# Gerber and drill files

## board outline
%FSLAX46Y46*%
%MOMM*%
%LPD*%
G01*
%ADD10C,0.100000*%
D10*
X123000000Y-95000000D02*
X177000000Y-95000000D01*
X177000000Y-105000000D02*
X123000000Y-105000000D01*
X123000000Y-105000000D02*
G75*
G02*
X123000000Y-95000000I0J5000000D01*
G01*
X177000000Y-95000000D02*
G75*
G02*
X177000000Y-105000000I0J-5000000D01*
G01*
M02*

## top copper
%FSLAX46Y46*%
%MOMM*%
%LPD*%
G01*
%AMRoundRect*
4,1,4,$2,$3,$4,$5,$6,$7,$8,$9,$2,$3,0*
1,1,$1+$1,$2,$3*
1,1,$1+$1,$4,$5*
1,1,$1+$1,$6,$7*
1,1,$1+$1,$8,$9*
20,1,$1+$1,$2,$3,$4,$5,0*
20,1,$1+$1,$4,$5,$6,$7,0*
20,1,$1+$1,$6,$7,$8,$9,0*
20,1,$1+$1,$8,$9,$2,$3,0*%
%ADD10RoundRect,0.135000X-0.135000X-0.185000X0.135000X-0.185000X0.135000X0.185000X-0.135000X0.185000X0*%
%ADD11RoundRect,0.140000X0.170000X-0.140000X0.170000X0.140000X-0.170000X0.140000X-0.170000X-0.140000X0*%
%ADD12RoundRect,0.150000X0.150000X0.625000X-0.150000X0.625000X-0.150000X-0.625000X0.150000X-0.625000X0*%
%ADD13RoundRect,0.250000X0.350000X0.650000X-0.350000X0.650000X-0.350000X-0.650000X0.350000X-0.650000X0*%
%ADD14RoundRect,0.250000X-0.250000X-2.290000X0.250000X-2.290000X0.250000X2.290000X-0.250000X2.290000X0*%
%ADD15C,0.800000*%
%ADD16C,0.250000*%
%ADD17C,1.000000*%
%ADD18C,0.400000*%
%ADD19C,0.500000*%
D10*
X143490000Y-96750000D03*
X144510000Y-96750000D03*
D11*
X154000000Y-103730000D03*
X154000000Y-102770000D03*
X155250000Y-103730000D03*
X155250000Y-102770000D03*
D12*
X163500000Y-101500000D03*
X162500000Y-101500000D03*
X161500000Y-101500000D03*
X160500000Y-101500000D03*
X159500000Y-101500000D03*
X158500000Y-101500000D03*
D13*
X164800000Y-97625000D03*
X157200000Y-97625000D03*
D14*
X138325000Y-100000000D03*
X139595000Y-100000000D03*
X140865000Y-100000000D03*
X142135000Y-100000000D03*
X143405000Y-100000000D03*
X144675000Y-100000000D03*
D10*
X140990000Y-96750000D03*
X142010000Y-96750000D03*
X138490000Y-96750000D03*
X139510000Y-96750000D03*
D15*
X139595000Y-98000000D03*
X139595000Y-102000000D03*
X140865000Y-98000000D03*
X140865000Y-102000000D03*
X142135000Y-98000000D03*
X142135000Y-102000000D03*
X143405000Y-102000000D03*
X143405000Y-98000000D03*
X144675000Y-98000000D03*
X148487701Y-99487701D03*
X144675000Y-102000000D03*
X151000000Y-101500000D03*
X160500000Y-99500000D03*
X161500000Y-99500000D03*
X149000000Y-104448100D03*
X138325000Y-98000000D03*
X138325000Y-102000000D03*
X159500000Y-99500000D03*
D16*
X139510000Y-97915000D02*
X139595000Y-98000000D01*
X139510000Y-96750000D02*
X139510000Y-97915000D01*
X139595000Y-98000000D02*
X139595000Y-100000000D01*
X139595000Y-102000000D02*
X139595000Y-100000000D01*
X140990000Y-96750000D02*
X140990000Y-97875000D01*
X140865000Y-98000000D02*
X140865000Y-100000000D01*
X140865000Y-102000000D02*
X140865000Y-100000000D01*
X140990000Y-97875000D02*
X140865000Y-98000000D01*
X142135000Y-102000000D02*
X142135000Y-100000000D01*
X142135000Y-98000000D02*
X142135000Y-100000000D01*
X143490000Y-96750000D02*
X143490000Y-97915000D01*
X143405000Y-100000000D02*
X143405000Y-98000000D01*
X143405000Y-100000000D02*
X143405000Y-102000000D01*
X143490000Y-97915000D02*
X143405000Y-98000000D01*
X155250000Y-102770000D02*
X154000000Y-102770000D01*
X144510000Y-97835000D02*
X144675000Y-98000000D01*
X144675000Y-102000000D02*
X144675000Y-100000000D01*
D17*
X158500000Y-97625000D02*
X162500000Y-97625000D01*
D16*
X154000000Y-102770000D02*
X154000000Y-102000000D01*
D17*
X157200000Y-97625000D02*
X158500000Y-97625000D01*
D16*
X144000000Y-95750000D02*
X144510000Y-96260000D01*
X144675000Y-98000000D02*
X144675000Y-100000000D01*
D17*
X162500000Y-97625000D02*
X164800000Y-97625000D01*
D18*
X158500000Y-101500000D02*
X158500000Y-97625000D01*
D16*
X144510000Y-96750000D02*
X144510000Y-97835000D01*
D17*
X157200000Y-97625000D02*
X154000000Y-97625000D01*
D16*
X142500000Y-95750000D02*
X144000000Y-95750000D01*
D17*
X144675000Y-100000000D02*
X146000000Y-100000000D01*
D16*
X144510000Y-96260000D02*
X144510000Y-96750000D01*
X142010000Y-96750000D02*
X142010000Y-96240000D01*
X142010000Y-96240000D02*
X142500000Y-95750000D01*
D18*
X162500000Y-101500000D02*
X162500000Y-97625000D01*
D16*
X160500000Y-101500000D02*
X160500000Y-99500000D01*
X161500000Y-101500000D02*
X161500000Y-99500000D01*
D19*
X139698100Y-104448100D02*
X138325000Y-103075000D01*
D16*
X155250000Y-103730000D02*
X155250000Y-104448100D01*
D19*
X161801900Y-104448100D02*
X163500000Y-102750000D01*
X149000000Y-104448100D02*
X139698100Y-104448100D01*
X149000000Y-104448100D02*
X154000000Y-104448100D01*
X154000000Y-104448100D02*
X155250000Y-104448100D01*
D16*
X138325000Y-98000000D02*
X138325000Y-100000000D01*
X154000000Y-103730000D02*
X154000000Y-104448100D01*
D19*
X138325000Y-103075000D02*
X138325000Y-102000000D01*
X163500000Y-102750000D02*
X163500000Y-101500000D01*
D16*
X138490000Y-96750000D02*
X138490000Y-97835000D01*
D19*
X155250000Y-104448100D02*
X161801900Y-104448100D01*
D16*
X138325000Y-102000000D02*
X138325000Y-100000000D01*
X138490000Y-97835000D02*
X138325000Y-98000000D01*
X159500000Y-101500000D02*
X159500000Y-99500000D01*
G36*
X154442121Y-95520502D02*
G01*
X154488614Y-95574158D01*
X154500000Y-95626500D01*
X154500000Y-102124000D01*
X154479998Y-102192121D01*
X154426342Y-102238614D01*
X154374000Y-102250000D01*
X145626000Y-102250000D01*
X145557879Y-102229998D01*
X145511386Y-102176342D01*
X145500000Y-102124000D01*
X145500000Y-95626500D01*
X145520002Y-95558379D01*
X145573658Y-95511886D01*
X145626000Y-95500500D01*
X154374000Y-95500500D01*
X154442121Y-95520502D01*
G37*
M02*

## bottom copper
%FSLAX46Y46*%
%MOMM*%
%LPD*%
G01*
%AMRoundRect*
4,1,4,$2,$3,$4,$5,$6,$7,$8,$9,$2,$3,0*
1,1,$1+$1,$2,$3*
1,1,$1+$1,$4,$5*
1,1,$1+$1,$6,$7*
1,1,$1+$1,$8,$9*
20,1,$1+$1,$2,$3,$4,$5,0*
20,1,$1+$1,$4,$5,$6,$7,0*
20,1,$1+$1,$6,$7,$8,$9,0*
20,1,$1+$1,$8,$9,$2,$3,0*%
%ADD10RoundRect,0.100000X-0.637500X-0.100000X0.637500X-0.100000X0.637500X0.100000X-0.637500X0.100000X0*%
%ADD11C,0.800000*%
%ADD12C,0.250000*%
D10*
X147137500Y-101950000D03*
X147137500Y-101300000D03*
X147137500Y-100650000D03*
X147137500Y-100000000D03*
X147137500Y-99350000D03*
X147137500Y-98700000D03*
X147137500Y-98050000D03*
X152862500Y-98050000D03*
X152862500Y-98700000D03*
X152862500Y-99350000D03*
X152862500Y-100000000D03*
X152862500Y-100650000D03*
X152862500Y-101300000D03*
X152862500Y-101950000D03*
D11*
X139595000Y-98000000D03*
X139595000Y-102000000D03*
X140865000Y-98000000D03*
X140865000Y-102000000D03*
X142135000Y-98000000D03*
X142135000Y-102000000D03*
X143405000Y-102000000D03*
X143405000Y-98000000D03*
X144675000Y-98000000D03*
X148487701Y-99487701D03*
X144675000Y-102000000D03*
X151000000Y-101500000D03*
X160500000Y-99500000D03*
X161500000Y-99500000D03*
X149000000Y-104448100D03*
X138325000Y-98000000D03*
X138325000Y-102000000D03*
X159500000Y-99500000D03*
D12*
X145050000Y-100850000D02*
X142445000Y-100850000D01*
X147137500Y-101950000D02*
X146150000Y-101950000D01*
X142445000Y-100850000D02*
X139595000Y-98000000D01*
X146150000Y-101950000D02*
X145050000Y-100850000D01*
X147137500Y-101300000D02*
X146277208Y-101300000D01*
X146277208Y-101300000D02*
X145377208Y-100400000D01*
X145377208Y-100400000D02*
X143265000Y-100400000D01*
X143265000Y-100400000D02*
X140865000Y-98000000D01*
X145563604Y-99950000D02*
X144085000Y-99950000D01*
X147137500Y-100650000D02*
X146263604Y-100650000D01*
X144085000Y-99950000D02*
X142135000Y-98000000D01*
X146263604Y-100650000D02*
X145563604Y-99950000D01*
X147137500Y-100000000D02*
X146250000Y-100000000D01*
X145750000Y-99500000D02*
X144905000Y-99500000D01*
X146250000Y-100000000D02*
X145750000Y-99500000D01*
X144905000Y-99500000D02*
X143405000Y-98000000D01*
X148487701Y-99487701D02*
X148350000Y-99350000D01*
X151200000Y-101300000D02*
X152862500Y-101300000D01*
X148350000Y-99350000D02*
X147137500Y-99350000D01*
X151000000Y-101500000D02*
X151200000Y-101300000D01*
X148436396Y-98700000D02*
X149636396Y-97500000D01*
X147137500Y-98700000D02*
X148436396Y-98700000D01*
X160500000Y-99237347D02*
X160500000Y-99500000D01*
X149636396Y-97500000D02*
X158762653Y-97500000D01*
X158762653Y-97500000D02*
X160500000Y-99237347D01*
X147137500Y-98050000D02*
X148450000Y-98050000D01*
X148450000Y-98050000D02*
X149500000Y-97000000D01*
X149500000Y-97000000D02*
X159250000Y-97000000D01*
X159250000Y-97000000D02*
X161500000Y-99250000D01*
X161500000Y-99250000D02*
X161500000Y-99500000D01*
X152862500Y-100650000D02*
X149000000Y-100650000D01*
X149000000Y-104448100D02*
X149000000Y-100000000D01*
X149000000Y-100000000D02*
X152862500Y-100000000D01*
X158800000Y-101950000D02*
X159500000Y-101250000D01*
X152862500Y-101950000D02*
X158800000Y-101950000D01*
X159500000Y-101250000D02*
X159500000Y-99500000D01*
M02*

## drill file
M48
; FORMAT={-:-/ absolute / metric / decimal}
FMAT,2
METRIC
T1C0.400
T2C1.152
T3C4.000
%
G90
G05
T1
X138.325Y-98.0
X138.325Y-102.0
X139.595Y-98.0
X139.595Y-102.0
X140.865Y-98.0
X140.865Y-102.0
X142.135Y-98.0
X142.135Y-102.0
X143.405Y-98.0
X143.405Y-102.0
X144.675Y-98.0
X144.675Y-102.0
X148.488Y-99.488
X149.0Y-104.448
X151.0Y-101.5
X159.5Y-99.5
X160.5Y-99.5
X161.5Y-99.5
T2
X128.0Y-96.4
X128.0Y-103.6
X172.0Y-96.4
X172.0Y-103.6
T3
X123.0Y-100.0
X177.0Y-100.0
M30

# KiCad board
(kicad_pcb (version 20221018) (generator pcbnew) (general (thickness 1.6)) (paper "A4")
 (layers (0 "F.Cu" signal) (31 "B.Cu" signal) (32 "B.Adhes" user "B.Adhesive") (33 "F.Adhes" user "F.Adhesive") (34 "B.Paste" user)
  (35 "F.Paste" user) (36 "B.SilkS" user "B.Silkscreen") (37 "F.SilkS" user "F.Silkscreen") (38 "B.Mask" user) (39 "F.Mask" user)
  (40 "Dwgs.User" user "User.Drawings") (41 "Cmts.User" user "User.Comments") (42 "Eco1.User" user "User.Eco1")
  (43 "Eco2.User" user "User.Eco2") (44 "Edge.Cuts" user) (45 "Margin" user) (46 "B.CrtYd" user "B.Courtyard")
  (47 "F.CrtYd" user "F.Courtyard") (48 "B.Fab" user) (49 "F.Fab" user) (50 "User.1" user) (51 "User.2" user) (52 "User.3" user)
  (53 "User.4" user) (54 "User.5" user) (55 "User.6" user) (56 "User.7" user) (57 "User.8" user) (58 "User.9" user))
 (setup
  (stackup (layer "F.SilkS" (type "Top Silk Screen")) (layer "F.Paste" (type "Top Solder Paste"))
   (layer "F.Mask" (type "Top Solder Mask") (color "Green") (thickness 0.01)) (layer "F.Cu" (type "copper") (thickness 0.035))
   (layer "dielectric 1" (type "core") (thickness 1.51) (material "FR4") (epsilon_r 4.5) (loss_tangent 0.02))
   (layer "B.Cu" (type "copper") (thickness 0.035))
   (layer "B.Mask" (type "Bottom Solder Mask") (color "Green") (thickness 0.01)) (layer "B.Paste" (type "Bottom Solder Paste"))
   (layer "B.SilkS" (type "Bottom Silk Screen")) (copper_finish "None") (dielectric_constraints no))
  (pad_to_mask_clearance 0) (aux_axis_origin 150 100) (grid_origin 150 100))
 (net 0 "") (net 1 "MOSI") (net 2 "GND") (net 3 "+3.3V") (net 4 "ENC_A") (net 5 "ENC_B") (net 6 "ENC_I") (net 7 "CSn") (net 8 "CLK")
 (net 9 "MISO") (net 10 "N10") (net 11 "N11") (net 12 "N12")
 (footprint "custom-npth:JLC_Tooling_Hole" (layer "F.Cu") (at 128 103.6)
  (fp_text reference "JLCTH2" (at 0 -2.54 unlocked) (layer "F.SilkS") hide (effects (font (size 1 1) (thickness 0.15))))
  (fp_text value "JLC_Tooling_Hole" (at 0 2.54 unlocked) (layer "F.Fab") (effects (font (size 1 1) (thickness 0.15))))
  (pad "" np_thru_hole circle (at 0 0) (size 1.3 1.3) (drill 1.152) (layers "*.Mask") (solder_mask_margin 0.074) (clearance 0.248)
   (zone_connect 0)))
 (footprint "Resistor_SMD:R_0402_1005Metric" (layer "F.Cu") (at 144 96.75)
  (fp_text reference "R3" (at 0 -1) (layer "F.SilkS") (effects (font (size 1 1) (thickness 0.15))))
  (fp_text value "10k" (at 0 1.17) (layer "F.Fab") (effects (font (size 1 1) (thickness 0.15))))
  (pad "1" smd roundrect (at -0.51 0) (size 0.54 0.64) (layers "F.Cu" "F.Paste" "F.Mask") (roundrect_rratio 0.25) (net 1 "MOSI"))
  (pad "2" smd roundrect (at 0.51 0) (size 0.54 0.64) (layers "F.Cu" "F.Paste" "F.Mask") (roundrect_rratio 0.25) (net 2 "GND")))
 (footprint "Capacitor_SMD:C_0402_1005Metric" (layer "F.Cu") (at 154 103.25 90)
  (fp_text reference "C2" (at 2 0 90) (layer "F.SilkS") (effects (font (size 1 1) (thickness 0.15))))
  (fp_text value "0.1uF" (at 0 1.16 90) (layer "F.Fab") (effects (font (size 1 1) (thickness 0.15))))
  (pad "1" smd roundrect (at -0.48 0 90) (size 0.56 0.62) (layers "F.Cu" "F.Paste" "F.Mask") (roundrect_rratio 0.25) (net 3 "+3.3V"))
  (pad "2" smd roundrect (at 0.48 0 90) (size 0.56 0.62) (layers "F.Cu" "F.Paste" "F.Mask") (roundrect_rratio 0.25) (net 2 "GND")))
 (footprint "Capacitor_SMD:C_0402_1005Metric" (layer "F.Cu") (at 155.25 103.25 90)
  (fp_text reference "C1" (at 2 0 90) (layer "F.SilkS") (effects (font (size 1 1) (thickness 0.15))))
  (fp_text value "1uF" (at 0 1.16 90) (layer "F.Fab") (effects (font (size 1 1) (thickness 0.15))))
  (pad "1" smd roundrect (at -0.48 0 90) (size 0.56 0.62) (layers "F.Cu" "F.Paste" "F.Mask") (roundrect_rratio 0.25) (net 3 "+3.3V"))
  (pad "2" smd roundrect (at 0.48 0 90) (size 0.56 0.62) (layers "F.Cu" "F.Paste" "F.Mask") (roundrect_rratio 0.25) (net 2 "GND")))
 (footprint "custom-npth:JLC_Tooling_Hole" (layer "F.Cu") (at 128 96.4)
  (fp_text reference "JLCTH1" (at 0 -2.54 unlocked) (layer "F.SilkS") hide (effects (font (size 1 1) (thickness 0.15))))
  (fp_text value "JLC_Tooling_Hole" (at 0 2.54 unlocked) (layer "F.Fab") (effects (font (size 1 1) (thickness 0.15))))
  (pad "" np_thru_hole circle (at 0 0) (size 1.3 1.3) (drill 1.152) (layers "*.Mask") (solder_mask_margin 0.074) (clearance 0.248)
   (zone_connect 0)))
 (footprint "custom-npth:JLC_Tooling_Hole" (layer "F.Cu") (at 172 103.6)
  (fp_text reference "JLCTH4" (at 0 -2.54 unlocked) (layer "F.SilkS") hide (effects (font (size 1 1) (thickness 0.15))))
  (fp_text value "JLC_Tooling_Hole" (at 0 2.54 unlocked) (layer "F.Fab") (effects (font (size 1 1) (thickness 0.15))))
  (pad "" np_thru_hole circle (at 0 0) (size 1.3 1.3) (drill 1.152) (layers "*.Mask") (solder_mask_margin 0.074) (clearance 0.248)
   (zone_connect 0)))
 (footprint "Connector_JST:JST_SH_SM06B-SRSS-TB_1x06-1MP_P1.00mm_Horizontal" (layer "F.Cu") (at 161 99.5 180)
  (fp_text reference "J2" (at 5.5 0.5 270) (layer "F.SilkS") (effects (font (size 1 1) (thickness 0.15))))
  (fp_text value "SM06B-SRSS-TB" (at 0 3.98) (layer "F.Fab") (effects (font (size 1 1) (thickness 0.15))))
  (pad "1" smd roundrect (at -2.5 -2 180) (size 0.6 1.55) (layers "F.Cu" "F.Paste" "F.Mask") (roundrect_rratio 0.25) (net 3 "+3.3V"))
  (pad "2" smd roundrect (at -1.5 -2 180) (size 0.6 1.55) (layers "F.Cu" "F.Paste" "F.Mask") (roundrect_rratio 0.25) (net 2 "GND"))
  (pad "3" smd roundrect (at -0.5 -2 180) (size 0.6 1.55) (layers "F.Cu" "F.Paste" "F.Mask") (roundrect_rratio 0.25) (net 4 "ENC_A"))
  (pad "4" smd roundrect (at 0.5 -2 180) (size 0.6 1.55) (layers "F.Cu" "F.Paste" "F.Mask") (roundrect_rratio 0.25) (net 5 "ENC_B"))
  (pad "5" smd roundrect (at 1.5 -2 180) (size 0.6 1.55) (layers "F.Cu" "F.Paste" "F.Mask") (roundrect_rratio 0.25) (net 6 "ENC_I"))
  (pad "6" smd roundrect (at 2.5 -2 180) (size 0.6 1.55) (layers "F.Cu" "F.Paste" "F.Mask") (roundrect_rratio 0.25) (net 2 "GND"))
  (pad "MP" smd roundrect (at -3.8 1.875 180) (size 1.2 1.8) (layers "F.Cu" "F.Paste" "F.Mask") (roundrect_rratio 0.2083333333)
   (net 2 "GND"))
  (pad "MP" smd roundrect (at 3.8 1.875 180) (size 1.2 1.8) (layers "F.Cu" "F.Paste" "F.Mask") (roundrect_rratio 0.2083333333) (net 2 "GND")))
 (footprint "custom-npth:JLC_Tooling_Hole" (layer "F.Cu") (at 172 96.4)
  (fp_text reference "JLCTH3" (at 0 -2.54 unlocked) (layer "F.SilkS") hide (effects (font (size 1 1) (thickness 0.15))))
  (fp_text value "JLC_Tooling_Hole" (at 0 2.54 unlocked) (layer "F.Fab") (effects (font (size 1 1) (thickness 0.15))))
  (pad "" np_thru_hole circle (at 0 0) (size 1.3 1.3) (drill 1.152) (layers "*.Mask") (solder_mask_margin 0.074) (clearance 0.248)
   (zone_connect 0)))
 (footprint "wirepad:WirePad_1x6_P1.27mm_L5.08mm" (layer "F.Cu") (at 141.5 100)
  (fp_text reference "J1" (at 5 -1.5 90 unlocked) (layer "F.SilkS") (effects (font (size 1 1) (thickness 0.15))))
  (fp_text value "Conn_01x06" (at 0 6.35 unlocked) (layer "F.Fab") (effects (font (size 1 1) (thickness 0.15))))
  (pad "1" smd roundrect (at -3.175 0) (size 1 5.08) (layers "F.Cu" "F.Paste" "F.Mask") (roundrect_rratio 0.25) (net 3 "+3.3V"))
  (pad "2" smd roundrect (at -1.905 0) (size 1 5.08) (layers "F.Cu" "F.Paste" "F.Mask") (roundrect_rratio 0.25) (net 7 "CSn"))
  (pad "3" smd roundrect (at -0.635 0) (size 1 5.08) (layers "F.Cu" "F.Paste" "F.Mask") (roundrect_rratio 0.25) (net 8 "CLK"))
  (pad "4" smd roundrect (at 0.635 0) (size 1 5.08) (layers "F.Cu" "F.Paste" "F.Mask") (roundrect_rratio 0.25) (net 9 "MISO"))
  (pad "5" smd roundrect (at 1.905 0) (size 1 5.08) (layers "F.Cu" "F.Paste" "F.Mask") (roundrect_rratio 0.25) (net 1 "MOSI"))
  (pad "6" smd roundrect (at 3.175 0) (size 1 5.08) (layers "F.Cu" "F.Paste" "F.Mask") (roundrect_rratio 0.25) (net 2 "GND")))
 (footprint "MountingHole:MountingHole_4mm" (layer "F.Cu") (at 123 100)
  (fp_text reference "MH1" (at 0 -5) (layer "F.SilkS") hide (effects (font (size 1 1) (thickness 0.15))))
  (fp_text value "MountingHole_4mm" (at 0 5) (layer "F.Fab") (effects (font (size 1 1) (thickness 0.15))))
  (pad "" np_thru_hole circle (at 0 0) (size 4 4) (drill 4) (layers "*.Cu" "*.Mask")))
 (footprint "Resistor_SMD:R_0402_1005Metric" (layer "F.Cu") (at 141.5 96.75)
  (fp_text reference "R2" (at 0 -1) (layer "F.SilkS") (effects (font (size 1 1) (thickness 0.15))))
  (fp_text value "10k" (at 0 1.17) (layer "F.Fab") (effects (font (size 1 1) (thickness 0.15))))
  (pad "1" smd roundrect (at -0.51 0) (size 0.54 0.64) (layers "F.Cu" "F.Paste" "F.Mask") (roundrect_rratio 0.25) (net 8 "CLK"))
  (pad "2" smd roundrect (at 0.51 0) (size 0.54 0.64) (layers "F.Cu" "F.Paste" "F.Mask") (roundrect_rratio 0.25) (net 2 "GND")))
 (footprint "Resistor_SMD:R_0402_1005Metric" (layer "F.Cu") (at 139 96.75)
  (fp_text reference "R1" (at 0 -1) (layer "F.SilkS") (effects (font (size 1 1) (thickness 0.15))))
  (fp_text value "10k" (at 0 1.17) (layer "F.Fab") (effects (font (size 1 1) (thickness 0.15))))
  (pad "1" smd roundrect (at -0.51 0) (size 0.54 0.64) (layers "F.Cu" "F.Paste" "F.Mask") (roundrect_rratio 0.25) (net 3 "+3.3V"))
  (pad "2" smd roundrect (at 0.51 0) (size 0.54 0.64) (layers "F.Cu" "F.Paste" "F.Mask") (roundrect_rratio 0.25) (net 7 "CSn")))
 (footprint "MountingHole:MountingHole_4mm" (layer "F.Cu") (at 177 100)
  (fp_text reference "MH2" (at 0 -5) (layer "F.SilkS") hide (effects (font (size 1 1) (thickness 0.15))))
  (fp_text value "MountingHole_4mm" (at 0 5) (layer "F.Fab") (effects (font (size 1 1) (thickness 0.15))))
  (pad "" np_thru_hole circle (at 0 0) (size 4 4) (drill 4) (layers "*.Cu" "*.Mask")))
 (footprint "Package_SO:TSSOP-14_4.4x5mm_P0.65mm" (layer "B.Cu") (at 150 100)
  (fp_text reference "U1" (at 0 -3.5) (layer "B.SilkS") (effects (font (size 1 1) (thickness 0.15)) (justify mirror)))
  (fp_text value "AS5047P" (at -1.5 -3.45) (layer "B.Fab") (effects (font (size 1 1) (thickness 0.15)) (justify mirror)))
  (pad "1" smd roundrect (at -2.8625 1.95) (size 1.475 0.4) (layers "B.Cu" "B.Paste" "B.Mask") (roundrect_rratio 0.25) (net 7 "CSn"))
  (pad "2" smd roundrect (at -2.8625 1.3) (size 1.475 0.4) (layers "B.Cu" "B.Paste" "B.Mask") (roundrect_rratio 0.25) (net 8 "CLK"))
  (pad "3" smd roundrect (at -2.8625 0.65) (size 1.475 0.4) (layers "B.Cu" "B.Paste" "B.Mask") (roundrect_rratio 0.25) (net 9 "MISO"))
  (pad "4" smd roundrect (at -2.8625 0) (size 1.475 0.4) (layers "B.Cu" "B.Paste" "B.Mask") (roundrect_rratio 0.25) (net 1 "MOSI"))
  (pad "5" smd roundrect (at -2.8625 -0.65) (size 1.475 0.4) (layers "B.Cu" "B.Paste" "B.Mask") (roundrect_rratio 0.25) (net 2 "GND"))
  (pad "6" smd roundrect (at -2.8625 -1.3) (size 1.475 0.4) (layers "B.Cu" "B.Paste" "B.Mask") (roundrect_rratio 0.25) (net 5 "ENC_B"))
  (pad "7" smd roundrect (at -2.8625 -1.95) (size 1.475 0.4) (layers "B.Cu" "B.Paste" "B.Mask") (roundrect_rratio 0.25) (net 4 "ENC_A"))
  (pad "8" smd roundrect (at 2.8625 -1.95) (size 1.475 0.4) (layers "B.Cu" "B.Paste" "B.Mask") (roundrect_rratio 0.25) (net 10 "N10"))
  (pad "9" smd roundrect (at 2.8625 -1.3) (size 1.475 0.4) (layers "B.Cu" "B.Paste" "B.Mask") (roundrect_rratio 0.25) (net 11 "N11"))
  (pad "10" smd roundrect (at 2.8625 -0.65) (size 1.475 0.4) (layers "B.Cu" "B.Paste" "B.Mask") (roundrect_rratio 0.25) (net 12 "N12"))
  (pad "11" smd roundrect (at 2.8625 0) (size 1.475 0.4) (layers "B.Cu" "B.Paste" "B.Mask") (roundrect_rratio 0.25) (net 3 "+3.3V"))
  (pad "12" smd roundrect (at 2.8625 0.65) (size 1.475 0.4) (layers "B.Cu" "B.Paste" "B.Mask") (roundrect_rratio 0.25) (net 3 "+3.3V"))
  (pad "13" smd roundrect (at 2.8625 1.3) (size 1.475 0.4) (layers "B.Cu" "B.Paste" "B.Mask") (roundrect_rratio 0.25) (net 2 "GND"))
  (pad "14" smd roundrect (at 2.8625 1.95) (size 1.475 0.4) (layers "B.Cu" "B.Paste" "B.Mask") (roundrect_rratio 0.25) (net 6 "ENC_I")))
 (gr_line (start 123 95) (end 177 95) (stroke (width 0.1) (type solid)) (layer "Edge.Cuts"))
 (gr_line (start 177 105) (end 123 105) (stroke (width 0.1) (type solid)) (layer "Edge.Cuts"))
 (gr_arc (start 123 105) (mid 118 100) (end 123 95) (stroke (width 0.1) (type solid)) (layer "Edge.Cuts"))
 (gr_arc (start 177 95) (mid 182 100) (end 177 105) (stroke (width 0.1) (type solid)) (layer "Edge.Cuts"))
 (segment (start 139.51 97.915) (end 139.595 98) (width 0.25) (layer "F.Cu") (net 7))
 (segment (start 139.51 96.75) (end 139.51 97.915) (width 0.25) (layer "F.Cu") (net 7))
 (segment (start 139.595 98) (end 139.595 100) (width 0.25) (layer "F.Cu") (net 7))
 (segment (start 139.595 102) (end 139.595 100) (width 0.25) (layer "F.Cu") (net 7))
 (via (at 139.595 98) (size 0.8) (drill 0.4) (layers "F.Cu" "B.Cu") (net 7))
 (via (at 139.595 102) (size 0.8) (drill 0.4) (layers "F.Cu" "B.Cu") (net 7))
 (segment (start 145.05 100.85) (end 142.445 100.85) (width 0.25) (layer "B.Cu") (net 7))
 (segment (start 147.1375 101.95) (end 146.15 101.95) (width 0.25) (layer "B.Cu") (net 7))
 (segment (start 142.445 100.85) (end 139.595 98) (width 0.25) (layer "B.Cu") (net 7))
 (segment (start 146.15 101.95) (end 145.05 100.85) (width 0.25) (layer "B.Cu") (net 7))
 (segment (start 140.99 96.75) (end 140.99 97.875) (width 0.25) (layer "F.Cu") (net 8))
 (segment (start 140.865 98) (end 140.865 100) (width 0.25) (layer "F.Cu") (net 8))
 (segment (start 140.865 102) (end 140.865 100) (width 0.25) (layer "F.Cu") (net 8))
 (segment (start 140.99 97.875) (end 140.865 98) (width 0.25) (layer "F.Cu") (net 8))
 (via (at 140.865 98) (size 0.8) (drill 0.4) (layers "F.Cu" "B.Cu") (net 8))
 (via (at 140.865 102) (size 0.8) (drill 0.4) (layers "F.Cu" "B.Cu") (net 8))
 (segment (start 147.1375 101.3) (end 146.277208 101.3) (width 0.25) (layer "B.Cu") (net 8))
 (segment (start 146.277208 101.3) (end 145.377208 100.4) (width 0.25) (layer "B.Cu") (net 8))
 (segment (start 145.377208 100.4) (end 143.265 100.4) (width 0.25) (layer "B.Cu") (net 8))
 (segment (start 143.265 100.4) (end 140.865 98) (width 0.25) (layer "B.Cu") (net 8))
 (segment (start 142.135 102) (end 142.135 100) (width 0.25) (layer "F.Cu") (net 9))
 (segment (start 142.135 98) (end 142.135 100) (width 0.25) (layer "F.Cu") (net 9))
 (via (at 142.135 98) (size 0.8) (drill 0.4) (layers "F.Cu" "B.Cu") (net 9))
 (via (at 142.135 102) (size 0.8) (drill 0.4) (layers "F.Cu" "B.Cu") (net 9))
 (segment (start 145.563604 99.95) (end 144.085 99.95) (width 0.25) (layer "B.Cu") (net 9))
 (segment (start 147.1375 100.65) (end 146.263604 100.65) (width 0.25) (layer "B.Cu") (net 9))
 (segment (start 144.085 99.95) (end 142.135 98) (width 0.25) (layer "B.Cu") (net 9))
 (segment (start 146.263604 100.65) (end 145.563604 99.95) (width 0.25) (layer "B.Cu") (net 9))
 (segment (start 143.49 96.75) (end 143.49 97.915) (width 0.25) (layer "F.Cu") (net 1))
 (segment (start 143.405 100) (end 143.405 98) (width 0.25) (layer "F.Cu") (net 1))
 (segment (start 143.405 100) (end 143.405 102) (width 0.25) (layer "F.Cu") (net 1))
 (segment (start 143.49 97.915) (end 143.405 98) (width 0.25) (layer "F.Cu") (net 1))
 (via (at 143.405 102) (size 0.8) (drill 0.4) (layers "F.Cu" "B.Cu") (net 1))
 (via (at 143.405 98) (size 0.8) (drill 0.4) (layers "F.Cu" "B.Cu") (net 1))
 (segment (start 147.1375 100) (end 146.25 100) (width 0.25) (layer "B.Cu") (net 1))
 (segment (start 145.75 99.5) (end 144.905 99.5) (width 0.25) (layer "B.Cu") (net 1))
 (segment (start 146.25 100) (end 145.75 99.5) (width 0.25) (layer "B.Cu") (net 1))
 (segment (start 144.905 99.5) (end 143.405 98) (width 0.25) (layer "B.Cu") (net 1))
 (segment (start 155.25 102.77) (end 154 102.77) (width 0.25) (layer "F.Cu") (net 2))
 (segment (start 144.51 97.835) (end 144.675 98) (width 0.25) (layer "F.Cu") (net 2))
 (segment (start 144.675 102) (end 144.675 100) (width 0.25) (layer "F.Cu") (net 2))
 (segment (start 158.5 97.625) (end 162.5 97.625) (width 1) (layer "F.Cu") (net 2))
 (segment (start 154 102.77) (end 154 102) (width 0.25) (layer "F.Cu") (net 2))
 (segment (start 157.2 97.625) (end 158.5 97.625) (width 1) (layer "F.Cu") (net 2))
 (segment (start 144 95.75) (end 144.51 96.26) (width 0.25) (layer "F.Cu") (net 2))
 (segment (start 144.675 98) (end 144.675 100) (width 0.25) (layer "F.Cu") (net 2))
 (segment (start 162.5 97.625) (end 164.8 97.625) (width 1) (layer "F.Cu") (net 2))
 (segment (start 158.5 101.5) (end 158.5 97.625) (width 0.4) (layer "F.Cu") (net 2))
 (segment (start 144.51 96.75) (end 144.51 97.835) (width 0.25) (layer "F.Cu") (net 2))
 (segment (start 157.2 97.625) (end 154 97.625) (width 1) (layer "F.Cu") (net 2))
 (segment (start 142.5 95.75) (end 144 95.75) (width 0.25) (layer "F.Cu") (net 2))
 (segment (start 144.675 100) (end 146 100) (width 1) (layer "F.Cu") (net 2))
 (segment (start 144.51 96.26) (end 144.51 96.75) (width 0.25) (layer "F.Cu") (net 2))
 (segment (start 142.01 96.75) (end 142.01 96.24) (width 0.25) (layer "F.Cu") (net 2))
 (segment (start 142.01 96.24) (end 142.5 95.75) (width 0.25) (layer "F.Cu") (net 2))
 (segment (start 162.5 101.5) (end 162.5 97.625) (width 0.4) (layer "F.Cu") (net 2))
 (via (at 144.675 98) (size 0.8) (drill 0.4) (layers "F.Cu" "B.Cu") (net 2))
 (via (at 148.487701 99.487701) (size 0.8) (drill 0.4) (layers "F.Cu" "B.Cu") (free) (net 2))
 (via (at 144.675 102) (size 0.8) (drill 0.4) (layers "F.Cu" "B.Cu") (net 2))
 (via (at 151 101.5) (size 0.8) (drill 0.4) (layers "F.Cu" "B.Cu") (free) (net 2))
 (segment (start 148.487701 99.487701) (end 148.35 99.35) (width 0.25) (layer "B.Cu") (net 2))
 (segment (start 151.2 101.3) (end 152.8625 101.3) (width 0.25) (layer "B.Cu") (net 2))
 (segment (start 148.35 99.35) (end 147.1375 99.35) (width 0.25) (layer "B.Cu") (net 2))
 (segment (start 151 101.5) (end 151.2 101.3) (width 0.25) (layer "B.Cu") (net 2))
 (segment (start 160.5 101.5) (end 160.5 99.5) (width 0.25) (layer "F.Cu") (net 5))
 (via (at 160.5 99.5) (size 0.8) (drill 0.4) (layers "F.Cu" "B.Cu") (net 5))
 (segment (start 148.436396 98.7) (end 149.636396 97.5) (width 0.25) (layer "B.Cu") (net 5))
 (segment (start 147.1375 98.7) (end 148.436396 98.7) (width 0.25) (layer "B.Cu") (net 5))
 (segment (start 160.5 99.237347) (end 160.5 99.5) (width 0.25) (layer "B.Cu") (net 5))
 (segment (start 149.636396 97.5) (end 158.762653 97.5) (width 0.25) (layer "B.Cu") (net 5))
 (segment (start 158.762653 97.5) (end 160.5 99.237347) (width 0.25) (layer "B.Cu") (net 5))
 (segment (start 161.5 101.5) (end 161.5 99.5) (width 0.25) (layer "F.Cu") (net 4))
 (via (at 161.5 99.5) (size 0.8) (drill 0.4) (layers "F.Cu" "B.Cu") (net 4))
 (segment (start 147.1375 98.05) (end 148.45 98.05) (width 0.25) (layer "B.Cu") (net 4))
 (segment (start 148.45 98.05) (end 149.5 97) (width 0.25) (layer "B.Cu") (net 4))
 (segment (start 149.5 97) (end 159.25 97) (width 0.25) (layer "B.Cu") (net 4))
 (segment (start 159.25 97) (end 161.5 99.25) (width 0.25) (layer "B.Cu") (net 4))
 (segment (start 161.5 99.25) (end 161.5 99.5) (width 0.25) (layer "B.Cu") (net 4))
 (segment (start 139.6981 104.4481) (end 138.325 103.075) (width 0.5) (layer "F.Cu") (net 3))
 (segment (start 155.25 103.73) (end 155.25 104.4481) (width 0.25) (layer "F.Cu") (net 3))
 (segment (start 161.8019 104.4481) (end 163.5 102.75) (width 0.5) (layer "F.Cu") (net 3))
 (segment (start 149 104.4481) (end 139.6981 104.4481) (width 0.5) (layer "F.Cu") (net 3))
 (segment (start 149 104.4481) (end 154 104.4481) (width 0.5) (layer "F.Cu") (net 3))
 (segment (start 154 104.4481) (end 155.25 104.4481) (width 0.5) (layer "F.Cu") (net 3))
 (segment (start 138.325 98) (end 138.325 100) (width 0.25) (layer "F.Cu") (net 3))
 (segment (start 154 103.73) (end 154 104.4481) (width 0.25) (layer "F.Cu") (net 3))
 (segment (start 138.325 103.075) (end 138.325 102) (width 0.5) (layer "F.Cu") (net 3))
 (segment (start 163.5 102.75) (end 163.5 101.5) (width 0.5) (layer "F.Cu") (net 3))
 (segment (start 138.49 96.75) (end 138.49 97.835) (width 0.25) (layer "F.Cu") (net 3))
 (segment (start 155.25 104.4481) (end 161.8019 104.4481) (width 0.5) (layer "F.Cu") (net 3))
 (segment (start 138.325 102) (end 138.325 100) (width 0.25) (layer "F.Cu") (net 3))
 (segment (start 138.49 97.835) (end 138.325 98) (width 0.25) (layer "F.Cu") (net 3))
 (via (at 149 104.4481) (size 0.8) (drill 0.4) (layers "F.Cu" "B.Cu") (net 3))
 (via (at 138.325 98) (size 0.8) (drill 0.4) (layers "F.Cu" "B.Cu") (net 3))
 (via (at 138.325 102) (size 0.8) (drill 0.4) (layers "F.Cu" "B.Cu") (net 3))
 (segment (start 152.8625 100.65) (end 149 100.65) (width 0.25) (layer "B.Cu") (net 3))
 (segment (start 149 104.4481) (end 149 100) (width 0.25) (layer "B.Cu") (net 3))
 (segment (start 149 100) (end 152.8625 100) (width 0.25) (layer "B.Cu") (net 3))
 (segment (start 159.5 101.5) (end 159.5 99.5) (width 0.25) (layer "F.Cu") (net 6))
 (via (at 159.5 99.5) (size 0.8) (drill 0.4) (layers "F.Cu" "B.Cu") (free) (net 6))
 (segment (start 158.8 101.95) (end 159.5 101.25) (width 0.25) (layer "B.Cu") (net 6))
 (segment (start 152.8625 101.95) (end 158.8 101.95) (width 0.25) (layer "B.Cu") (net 6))
 (segment (start 159.5 101.25) (end 159.5 99.5) (width 0.25) (layer "B.Cu") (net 6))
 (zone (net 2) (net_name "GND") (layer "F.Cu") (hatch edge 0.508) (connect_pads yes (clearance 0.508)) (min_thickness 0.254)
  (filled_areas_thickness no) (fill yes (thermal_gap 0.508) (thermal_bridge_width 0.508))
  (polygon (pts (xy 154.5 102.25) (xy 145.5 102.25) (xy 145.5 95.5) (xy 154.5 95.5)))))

